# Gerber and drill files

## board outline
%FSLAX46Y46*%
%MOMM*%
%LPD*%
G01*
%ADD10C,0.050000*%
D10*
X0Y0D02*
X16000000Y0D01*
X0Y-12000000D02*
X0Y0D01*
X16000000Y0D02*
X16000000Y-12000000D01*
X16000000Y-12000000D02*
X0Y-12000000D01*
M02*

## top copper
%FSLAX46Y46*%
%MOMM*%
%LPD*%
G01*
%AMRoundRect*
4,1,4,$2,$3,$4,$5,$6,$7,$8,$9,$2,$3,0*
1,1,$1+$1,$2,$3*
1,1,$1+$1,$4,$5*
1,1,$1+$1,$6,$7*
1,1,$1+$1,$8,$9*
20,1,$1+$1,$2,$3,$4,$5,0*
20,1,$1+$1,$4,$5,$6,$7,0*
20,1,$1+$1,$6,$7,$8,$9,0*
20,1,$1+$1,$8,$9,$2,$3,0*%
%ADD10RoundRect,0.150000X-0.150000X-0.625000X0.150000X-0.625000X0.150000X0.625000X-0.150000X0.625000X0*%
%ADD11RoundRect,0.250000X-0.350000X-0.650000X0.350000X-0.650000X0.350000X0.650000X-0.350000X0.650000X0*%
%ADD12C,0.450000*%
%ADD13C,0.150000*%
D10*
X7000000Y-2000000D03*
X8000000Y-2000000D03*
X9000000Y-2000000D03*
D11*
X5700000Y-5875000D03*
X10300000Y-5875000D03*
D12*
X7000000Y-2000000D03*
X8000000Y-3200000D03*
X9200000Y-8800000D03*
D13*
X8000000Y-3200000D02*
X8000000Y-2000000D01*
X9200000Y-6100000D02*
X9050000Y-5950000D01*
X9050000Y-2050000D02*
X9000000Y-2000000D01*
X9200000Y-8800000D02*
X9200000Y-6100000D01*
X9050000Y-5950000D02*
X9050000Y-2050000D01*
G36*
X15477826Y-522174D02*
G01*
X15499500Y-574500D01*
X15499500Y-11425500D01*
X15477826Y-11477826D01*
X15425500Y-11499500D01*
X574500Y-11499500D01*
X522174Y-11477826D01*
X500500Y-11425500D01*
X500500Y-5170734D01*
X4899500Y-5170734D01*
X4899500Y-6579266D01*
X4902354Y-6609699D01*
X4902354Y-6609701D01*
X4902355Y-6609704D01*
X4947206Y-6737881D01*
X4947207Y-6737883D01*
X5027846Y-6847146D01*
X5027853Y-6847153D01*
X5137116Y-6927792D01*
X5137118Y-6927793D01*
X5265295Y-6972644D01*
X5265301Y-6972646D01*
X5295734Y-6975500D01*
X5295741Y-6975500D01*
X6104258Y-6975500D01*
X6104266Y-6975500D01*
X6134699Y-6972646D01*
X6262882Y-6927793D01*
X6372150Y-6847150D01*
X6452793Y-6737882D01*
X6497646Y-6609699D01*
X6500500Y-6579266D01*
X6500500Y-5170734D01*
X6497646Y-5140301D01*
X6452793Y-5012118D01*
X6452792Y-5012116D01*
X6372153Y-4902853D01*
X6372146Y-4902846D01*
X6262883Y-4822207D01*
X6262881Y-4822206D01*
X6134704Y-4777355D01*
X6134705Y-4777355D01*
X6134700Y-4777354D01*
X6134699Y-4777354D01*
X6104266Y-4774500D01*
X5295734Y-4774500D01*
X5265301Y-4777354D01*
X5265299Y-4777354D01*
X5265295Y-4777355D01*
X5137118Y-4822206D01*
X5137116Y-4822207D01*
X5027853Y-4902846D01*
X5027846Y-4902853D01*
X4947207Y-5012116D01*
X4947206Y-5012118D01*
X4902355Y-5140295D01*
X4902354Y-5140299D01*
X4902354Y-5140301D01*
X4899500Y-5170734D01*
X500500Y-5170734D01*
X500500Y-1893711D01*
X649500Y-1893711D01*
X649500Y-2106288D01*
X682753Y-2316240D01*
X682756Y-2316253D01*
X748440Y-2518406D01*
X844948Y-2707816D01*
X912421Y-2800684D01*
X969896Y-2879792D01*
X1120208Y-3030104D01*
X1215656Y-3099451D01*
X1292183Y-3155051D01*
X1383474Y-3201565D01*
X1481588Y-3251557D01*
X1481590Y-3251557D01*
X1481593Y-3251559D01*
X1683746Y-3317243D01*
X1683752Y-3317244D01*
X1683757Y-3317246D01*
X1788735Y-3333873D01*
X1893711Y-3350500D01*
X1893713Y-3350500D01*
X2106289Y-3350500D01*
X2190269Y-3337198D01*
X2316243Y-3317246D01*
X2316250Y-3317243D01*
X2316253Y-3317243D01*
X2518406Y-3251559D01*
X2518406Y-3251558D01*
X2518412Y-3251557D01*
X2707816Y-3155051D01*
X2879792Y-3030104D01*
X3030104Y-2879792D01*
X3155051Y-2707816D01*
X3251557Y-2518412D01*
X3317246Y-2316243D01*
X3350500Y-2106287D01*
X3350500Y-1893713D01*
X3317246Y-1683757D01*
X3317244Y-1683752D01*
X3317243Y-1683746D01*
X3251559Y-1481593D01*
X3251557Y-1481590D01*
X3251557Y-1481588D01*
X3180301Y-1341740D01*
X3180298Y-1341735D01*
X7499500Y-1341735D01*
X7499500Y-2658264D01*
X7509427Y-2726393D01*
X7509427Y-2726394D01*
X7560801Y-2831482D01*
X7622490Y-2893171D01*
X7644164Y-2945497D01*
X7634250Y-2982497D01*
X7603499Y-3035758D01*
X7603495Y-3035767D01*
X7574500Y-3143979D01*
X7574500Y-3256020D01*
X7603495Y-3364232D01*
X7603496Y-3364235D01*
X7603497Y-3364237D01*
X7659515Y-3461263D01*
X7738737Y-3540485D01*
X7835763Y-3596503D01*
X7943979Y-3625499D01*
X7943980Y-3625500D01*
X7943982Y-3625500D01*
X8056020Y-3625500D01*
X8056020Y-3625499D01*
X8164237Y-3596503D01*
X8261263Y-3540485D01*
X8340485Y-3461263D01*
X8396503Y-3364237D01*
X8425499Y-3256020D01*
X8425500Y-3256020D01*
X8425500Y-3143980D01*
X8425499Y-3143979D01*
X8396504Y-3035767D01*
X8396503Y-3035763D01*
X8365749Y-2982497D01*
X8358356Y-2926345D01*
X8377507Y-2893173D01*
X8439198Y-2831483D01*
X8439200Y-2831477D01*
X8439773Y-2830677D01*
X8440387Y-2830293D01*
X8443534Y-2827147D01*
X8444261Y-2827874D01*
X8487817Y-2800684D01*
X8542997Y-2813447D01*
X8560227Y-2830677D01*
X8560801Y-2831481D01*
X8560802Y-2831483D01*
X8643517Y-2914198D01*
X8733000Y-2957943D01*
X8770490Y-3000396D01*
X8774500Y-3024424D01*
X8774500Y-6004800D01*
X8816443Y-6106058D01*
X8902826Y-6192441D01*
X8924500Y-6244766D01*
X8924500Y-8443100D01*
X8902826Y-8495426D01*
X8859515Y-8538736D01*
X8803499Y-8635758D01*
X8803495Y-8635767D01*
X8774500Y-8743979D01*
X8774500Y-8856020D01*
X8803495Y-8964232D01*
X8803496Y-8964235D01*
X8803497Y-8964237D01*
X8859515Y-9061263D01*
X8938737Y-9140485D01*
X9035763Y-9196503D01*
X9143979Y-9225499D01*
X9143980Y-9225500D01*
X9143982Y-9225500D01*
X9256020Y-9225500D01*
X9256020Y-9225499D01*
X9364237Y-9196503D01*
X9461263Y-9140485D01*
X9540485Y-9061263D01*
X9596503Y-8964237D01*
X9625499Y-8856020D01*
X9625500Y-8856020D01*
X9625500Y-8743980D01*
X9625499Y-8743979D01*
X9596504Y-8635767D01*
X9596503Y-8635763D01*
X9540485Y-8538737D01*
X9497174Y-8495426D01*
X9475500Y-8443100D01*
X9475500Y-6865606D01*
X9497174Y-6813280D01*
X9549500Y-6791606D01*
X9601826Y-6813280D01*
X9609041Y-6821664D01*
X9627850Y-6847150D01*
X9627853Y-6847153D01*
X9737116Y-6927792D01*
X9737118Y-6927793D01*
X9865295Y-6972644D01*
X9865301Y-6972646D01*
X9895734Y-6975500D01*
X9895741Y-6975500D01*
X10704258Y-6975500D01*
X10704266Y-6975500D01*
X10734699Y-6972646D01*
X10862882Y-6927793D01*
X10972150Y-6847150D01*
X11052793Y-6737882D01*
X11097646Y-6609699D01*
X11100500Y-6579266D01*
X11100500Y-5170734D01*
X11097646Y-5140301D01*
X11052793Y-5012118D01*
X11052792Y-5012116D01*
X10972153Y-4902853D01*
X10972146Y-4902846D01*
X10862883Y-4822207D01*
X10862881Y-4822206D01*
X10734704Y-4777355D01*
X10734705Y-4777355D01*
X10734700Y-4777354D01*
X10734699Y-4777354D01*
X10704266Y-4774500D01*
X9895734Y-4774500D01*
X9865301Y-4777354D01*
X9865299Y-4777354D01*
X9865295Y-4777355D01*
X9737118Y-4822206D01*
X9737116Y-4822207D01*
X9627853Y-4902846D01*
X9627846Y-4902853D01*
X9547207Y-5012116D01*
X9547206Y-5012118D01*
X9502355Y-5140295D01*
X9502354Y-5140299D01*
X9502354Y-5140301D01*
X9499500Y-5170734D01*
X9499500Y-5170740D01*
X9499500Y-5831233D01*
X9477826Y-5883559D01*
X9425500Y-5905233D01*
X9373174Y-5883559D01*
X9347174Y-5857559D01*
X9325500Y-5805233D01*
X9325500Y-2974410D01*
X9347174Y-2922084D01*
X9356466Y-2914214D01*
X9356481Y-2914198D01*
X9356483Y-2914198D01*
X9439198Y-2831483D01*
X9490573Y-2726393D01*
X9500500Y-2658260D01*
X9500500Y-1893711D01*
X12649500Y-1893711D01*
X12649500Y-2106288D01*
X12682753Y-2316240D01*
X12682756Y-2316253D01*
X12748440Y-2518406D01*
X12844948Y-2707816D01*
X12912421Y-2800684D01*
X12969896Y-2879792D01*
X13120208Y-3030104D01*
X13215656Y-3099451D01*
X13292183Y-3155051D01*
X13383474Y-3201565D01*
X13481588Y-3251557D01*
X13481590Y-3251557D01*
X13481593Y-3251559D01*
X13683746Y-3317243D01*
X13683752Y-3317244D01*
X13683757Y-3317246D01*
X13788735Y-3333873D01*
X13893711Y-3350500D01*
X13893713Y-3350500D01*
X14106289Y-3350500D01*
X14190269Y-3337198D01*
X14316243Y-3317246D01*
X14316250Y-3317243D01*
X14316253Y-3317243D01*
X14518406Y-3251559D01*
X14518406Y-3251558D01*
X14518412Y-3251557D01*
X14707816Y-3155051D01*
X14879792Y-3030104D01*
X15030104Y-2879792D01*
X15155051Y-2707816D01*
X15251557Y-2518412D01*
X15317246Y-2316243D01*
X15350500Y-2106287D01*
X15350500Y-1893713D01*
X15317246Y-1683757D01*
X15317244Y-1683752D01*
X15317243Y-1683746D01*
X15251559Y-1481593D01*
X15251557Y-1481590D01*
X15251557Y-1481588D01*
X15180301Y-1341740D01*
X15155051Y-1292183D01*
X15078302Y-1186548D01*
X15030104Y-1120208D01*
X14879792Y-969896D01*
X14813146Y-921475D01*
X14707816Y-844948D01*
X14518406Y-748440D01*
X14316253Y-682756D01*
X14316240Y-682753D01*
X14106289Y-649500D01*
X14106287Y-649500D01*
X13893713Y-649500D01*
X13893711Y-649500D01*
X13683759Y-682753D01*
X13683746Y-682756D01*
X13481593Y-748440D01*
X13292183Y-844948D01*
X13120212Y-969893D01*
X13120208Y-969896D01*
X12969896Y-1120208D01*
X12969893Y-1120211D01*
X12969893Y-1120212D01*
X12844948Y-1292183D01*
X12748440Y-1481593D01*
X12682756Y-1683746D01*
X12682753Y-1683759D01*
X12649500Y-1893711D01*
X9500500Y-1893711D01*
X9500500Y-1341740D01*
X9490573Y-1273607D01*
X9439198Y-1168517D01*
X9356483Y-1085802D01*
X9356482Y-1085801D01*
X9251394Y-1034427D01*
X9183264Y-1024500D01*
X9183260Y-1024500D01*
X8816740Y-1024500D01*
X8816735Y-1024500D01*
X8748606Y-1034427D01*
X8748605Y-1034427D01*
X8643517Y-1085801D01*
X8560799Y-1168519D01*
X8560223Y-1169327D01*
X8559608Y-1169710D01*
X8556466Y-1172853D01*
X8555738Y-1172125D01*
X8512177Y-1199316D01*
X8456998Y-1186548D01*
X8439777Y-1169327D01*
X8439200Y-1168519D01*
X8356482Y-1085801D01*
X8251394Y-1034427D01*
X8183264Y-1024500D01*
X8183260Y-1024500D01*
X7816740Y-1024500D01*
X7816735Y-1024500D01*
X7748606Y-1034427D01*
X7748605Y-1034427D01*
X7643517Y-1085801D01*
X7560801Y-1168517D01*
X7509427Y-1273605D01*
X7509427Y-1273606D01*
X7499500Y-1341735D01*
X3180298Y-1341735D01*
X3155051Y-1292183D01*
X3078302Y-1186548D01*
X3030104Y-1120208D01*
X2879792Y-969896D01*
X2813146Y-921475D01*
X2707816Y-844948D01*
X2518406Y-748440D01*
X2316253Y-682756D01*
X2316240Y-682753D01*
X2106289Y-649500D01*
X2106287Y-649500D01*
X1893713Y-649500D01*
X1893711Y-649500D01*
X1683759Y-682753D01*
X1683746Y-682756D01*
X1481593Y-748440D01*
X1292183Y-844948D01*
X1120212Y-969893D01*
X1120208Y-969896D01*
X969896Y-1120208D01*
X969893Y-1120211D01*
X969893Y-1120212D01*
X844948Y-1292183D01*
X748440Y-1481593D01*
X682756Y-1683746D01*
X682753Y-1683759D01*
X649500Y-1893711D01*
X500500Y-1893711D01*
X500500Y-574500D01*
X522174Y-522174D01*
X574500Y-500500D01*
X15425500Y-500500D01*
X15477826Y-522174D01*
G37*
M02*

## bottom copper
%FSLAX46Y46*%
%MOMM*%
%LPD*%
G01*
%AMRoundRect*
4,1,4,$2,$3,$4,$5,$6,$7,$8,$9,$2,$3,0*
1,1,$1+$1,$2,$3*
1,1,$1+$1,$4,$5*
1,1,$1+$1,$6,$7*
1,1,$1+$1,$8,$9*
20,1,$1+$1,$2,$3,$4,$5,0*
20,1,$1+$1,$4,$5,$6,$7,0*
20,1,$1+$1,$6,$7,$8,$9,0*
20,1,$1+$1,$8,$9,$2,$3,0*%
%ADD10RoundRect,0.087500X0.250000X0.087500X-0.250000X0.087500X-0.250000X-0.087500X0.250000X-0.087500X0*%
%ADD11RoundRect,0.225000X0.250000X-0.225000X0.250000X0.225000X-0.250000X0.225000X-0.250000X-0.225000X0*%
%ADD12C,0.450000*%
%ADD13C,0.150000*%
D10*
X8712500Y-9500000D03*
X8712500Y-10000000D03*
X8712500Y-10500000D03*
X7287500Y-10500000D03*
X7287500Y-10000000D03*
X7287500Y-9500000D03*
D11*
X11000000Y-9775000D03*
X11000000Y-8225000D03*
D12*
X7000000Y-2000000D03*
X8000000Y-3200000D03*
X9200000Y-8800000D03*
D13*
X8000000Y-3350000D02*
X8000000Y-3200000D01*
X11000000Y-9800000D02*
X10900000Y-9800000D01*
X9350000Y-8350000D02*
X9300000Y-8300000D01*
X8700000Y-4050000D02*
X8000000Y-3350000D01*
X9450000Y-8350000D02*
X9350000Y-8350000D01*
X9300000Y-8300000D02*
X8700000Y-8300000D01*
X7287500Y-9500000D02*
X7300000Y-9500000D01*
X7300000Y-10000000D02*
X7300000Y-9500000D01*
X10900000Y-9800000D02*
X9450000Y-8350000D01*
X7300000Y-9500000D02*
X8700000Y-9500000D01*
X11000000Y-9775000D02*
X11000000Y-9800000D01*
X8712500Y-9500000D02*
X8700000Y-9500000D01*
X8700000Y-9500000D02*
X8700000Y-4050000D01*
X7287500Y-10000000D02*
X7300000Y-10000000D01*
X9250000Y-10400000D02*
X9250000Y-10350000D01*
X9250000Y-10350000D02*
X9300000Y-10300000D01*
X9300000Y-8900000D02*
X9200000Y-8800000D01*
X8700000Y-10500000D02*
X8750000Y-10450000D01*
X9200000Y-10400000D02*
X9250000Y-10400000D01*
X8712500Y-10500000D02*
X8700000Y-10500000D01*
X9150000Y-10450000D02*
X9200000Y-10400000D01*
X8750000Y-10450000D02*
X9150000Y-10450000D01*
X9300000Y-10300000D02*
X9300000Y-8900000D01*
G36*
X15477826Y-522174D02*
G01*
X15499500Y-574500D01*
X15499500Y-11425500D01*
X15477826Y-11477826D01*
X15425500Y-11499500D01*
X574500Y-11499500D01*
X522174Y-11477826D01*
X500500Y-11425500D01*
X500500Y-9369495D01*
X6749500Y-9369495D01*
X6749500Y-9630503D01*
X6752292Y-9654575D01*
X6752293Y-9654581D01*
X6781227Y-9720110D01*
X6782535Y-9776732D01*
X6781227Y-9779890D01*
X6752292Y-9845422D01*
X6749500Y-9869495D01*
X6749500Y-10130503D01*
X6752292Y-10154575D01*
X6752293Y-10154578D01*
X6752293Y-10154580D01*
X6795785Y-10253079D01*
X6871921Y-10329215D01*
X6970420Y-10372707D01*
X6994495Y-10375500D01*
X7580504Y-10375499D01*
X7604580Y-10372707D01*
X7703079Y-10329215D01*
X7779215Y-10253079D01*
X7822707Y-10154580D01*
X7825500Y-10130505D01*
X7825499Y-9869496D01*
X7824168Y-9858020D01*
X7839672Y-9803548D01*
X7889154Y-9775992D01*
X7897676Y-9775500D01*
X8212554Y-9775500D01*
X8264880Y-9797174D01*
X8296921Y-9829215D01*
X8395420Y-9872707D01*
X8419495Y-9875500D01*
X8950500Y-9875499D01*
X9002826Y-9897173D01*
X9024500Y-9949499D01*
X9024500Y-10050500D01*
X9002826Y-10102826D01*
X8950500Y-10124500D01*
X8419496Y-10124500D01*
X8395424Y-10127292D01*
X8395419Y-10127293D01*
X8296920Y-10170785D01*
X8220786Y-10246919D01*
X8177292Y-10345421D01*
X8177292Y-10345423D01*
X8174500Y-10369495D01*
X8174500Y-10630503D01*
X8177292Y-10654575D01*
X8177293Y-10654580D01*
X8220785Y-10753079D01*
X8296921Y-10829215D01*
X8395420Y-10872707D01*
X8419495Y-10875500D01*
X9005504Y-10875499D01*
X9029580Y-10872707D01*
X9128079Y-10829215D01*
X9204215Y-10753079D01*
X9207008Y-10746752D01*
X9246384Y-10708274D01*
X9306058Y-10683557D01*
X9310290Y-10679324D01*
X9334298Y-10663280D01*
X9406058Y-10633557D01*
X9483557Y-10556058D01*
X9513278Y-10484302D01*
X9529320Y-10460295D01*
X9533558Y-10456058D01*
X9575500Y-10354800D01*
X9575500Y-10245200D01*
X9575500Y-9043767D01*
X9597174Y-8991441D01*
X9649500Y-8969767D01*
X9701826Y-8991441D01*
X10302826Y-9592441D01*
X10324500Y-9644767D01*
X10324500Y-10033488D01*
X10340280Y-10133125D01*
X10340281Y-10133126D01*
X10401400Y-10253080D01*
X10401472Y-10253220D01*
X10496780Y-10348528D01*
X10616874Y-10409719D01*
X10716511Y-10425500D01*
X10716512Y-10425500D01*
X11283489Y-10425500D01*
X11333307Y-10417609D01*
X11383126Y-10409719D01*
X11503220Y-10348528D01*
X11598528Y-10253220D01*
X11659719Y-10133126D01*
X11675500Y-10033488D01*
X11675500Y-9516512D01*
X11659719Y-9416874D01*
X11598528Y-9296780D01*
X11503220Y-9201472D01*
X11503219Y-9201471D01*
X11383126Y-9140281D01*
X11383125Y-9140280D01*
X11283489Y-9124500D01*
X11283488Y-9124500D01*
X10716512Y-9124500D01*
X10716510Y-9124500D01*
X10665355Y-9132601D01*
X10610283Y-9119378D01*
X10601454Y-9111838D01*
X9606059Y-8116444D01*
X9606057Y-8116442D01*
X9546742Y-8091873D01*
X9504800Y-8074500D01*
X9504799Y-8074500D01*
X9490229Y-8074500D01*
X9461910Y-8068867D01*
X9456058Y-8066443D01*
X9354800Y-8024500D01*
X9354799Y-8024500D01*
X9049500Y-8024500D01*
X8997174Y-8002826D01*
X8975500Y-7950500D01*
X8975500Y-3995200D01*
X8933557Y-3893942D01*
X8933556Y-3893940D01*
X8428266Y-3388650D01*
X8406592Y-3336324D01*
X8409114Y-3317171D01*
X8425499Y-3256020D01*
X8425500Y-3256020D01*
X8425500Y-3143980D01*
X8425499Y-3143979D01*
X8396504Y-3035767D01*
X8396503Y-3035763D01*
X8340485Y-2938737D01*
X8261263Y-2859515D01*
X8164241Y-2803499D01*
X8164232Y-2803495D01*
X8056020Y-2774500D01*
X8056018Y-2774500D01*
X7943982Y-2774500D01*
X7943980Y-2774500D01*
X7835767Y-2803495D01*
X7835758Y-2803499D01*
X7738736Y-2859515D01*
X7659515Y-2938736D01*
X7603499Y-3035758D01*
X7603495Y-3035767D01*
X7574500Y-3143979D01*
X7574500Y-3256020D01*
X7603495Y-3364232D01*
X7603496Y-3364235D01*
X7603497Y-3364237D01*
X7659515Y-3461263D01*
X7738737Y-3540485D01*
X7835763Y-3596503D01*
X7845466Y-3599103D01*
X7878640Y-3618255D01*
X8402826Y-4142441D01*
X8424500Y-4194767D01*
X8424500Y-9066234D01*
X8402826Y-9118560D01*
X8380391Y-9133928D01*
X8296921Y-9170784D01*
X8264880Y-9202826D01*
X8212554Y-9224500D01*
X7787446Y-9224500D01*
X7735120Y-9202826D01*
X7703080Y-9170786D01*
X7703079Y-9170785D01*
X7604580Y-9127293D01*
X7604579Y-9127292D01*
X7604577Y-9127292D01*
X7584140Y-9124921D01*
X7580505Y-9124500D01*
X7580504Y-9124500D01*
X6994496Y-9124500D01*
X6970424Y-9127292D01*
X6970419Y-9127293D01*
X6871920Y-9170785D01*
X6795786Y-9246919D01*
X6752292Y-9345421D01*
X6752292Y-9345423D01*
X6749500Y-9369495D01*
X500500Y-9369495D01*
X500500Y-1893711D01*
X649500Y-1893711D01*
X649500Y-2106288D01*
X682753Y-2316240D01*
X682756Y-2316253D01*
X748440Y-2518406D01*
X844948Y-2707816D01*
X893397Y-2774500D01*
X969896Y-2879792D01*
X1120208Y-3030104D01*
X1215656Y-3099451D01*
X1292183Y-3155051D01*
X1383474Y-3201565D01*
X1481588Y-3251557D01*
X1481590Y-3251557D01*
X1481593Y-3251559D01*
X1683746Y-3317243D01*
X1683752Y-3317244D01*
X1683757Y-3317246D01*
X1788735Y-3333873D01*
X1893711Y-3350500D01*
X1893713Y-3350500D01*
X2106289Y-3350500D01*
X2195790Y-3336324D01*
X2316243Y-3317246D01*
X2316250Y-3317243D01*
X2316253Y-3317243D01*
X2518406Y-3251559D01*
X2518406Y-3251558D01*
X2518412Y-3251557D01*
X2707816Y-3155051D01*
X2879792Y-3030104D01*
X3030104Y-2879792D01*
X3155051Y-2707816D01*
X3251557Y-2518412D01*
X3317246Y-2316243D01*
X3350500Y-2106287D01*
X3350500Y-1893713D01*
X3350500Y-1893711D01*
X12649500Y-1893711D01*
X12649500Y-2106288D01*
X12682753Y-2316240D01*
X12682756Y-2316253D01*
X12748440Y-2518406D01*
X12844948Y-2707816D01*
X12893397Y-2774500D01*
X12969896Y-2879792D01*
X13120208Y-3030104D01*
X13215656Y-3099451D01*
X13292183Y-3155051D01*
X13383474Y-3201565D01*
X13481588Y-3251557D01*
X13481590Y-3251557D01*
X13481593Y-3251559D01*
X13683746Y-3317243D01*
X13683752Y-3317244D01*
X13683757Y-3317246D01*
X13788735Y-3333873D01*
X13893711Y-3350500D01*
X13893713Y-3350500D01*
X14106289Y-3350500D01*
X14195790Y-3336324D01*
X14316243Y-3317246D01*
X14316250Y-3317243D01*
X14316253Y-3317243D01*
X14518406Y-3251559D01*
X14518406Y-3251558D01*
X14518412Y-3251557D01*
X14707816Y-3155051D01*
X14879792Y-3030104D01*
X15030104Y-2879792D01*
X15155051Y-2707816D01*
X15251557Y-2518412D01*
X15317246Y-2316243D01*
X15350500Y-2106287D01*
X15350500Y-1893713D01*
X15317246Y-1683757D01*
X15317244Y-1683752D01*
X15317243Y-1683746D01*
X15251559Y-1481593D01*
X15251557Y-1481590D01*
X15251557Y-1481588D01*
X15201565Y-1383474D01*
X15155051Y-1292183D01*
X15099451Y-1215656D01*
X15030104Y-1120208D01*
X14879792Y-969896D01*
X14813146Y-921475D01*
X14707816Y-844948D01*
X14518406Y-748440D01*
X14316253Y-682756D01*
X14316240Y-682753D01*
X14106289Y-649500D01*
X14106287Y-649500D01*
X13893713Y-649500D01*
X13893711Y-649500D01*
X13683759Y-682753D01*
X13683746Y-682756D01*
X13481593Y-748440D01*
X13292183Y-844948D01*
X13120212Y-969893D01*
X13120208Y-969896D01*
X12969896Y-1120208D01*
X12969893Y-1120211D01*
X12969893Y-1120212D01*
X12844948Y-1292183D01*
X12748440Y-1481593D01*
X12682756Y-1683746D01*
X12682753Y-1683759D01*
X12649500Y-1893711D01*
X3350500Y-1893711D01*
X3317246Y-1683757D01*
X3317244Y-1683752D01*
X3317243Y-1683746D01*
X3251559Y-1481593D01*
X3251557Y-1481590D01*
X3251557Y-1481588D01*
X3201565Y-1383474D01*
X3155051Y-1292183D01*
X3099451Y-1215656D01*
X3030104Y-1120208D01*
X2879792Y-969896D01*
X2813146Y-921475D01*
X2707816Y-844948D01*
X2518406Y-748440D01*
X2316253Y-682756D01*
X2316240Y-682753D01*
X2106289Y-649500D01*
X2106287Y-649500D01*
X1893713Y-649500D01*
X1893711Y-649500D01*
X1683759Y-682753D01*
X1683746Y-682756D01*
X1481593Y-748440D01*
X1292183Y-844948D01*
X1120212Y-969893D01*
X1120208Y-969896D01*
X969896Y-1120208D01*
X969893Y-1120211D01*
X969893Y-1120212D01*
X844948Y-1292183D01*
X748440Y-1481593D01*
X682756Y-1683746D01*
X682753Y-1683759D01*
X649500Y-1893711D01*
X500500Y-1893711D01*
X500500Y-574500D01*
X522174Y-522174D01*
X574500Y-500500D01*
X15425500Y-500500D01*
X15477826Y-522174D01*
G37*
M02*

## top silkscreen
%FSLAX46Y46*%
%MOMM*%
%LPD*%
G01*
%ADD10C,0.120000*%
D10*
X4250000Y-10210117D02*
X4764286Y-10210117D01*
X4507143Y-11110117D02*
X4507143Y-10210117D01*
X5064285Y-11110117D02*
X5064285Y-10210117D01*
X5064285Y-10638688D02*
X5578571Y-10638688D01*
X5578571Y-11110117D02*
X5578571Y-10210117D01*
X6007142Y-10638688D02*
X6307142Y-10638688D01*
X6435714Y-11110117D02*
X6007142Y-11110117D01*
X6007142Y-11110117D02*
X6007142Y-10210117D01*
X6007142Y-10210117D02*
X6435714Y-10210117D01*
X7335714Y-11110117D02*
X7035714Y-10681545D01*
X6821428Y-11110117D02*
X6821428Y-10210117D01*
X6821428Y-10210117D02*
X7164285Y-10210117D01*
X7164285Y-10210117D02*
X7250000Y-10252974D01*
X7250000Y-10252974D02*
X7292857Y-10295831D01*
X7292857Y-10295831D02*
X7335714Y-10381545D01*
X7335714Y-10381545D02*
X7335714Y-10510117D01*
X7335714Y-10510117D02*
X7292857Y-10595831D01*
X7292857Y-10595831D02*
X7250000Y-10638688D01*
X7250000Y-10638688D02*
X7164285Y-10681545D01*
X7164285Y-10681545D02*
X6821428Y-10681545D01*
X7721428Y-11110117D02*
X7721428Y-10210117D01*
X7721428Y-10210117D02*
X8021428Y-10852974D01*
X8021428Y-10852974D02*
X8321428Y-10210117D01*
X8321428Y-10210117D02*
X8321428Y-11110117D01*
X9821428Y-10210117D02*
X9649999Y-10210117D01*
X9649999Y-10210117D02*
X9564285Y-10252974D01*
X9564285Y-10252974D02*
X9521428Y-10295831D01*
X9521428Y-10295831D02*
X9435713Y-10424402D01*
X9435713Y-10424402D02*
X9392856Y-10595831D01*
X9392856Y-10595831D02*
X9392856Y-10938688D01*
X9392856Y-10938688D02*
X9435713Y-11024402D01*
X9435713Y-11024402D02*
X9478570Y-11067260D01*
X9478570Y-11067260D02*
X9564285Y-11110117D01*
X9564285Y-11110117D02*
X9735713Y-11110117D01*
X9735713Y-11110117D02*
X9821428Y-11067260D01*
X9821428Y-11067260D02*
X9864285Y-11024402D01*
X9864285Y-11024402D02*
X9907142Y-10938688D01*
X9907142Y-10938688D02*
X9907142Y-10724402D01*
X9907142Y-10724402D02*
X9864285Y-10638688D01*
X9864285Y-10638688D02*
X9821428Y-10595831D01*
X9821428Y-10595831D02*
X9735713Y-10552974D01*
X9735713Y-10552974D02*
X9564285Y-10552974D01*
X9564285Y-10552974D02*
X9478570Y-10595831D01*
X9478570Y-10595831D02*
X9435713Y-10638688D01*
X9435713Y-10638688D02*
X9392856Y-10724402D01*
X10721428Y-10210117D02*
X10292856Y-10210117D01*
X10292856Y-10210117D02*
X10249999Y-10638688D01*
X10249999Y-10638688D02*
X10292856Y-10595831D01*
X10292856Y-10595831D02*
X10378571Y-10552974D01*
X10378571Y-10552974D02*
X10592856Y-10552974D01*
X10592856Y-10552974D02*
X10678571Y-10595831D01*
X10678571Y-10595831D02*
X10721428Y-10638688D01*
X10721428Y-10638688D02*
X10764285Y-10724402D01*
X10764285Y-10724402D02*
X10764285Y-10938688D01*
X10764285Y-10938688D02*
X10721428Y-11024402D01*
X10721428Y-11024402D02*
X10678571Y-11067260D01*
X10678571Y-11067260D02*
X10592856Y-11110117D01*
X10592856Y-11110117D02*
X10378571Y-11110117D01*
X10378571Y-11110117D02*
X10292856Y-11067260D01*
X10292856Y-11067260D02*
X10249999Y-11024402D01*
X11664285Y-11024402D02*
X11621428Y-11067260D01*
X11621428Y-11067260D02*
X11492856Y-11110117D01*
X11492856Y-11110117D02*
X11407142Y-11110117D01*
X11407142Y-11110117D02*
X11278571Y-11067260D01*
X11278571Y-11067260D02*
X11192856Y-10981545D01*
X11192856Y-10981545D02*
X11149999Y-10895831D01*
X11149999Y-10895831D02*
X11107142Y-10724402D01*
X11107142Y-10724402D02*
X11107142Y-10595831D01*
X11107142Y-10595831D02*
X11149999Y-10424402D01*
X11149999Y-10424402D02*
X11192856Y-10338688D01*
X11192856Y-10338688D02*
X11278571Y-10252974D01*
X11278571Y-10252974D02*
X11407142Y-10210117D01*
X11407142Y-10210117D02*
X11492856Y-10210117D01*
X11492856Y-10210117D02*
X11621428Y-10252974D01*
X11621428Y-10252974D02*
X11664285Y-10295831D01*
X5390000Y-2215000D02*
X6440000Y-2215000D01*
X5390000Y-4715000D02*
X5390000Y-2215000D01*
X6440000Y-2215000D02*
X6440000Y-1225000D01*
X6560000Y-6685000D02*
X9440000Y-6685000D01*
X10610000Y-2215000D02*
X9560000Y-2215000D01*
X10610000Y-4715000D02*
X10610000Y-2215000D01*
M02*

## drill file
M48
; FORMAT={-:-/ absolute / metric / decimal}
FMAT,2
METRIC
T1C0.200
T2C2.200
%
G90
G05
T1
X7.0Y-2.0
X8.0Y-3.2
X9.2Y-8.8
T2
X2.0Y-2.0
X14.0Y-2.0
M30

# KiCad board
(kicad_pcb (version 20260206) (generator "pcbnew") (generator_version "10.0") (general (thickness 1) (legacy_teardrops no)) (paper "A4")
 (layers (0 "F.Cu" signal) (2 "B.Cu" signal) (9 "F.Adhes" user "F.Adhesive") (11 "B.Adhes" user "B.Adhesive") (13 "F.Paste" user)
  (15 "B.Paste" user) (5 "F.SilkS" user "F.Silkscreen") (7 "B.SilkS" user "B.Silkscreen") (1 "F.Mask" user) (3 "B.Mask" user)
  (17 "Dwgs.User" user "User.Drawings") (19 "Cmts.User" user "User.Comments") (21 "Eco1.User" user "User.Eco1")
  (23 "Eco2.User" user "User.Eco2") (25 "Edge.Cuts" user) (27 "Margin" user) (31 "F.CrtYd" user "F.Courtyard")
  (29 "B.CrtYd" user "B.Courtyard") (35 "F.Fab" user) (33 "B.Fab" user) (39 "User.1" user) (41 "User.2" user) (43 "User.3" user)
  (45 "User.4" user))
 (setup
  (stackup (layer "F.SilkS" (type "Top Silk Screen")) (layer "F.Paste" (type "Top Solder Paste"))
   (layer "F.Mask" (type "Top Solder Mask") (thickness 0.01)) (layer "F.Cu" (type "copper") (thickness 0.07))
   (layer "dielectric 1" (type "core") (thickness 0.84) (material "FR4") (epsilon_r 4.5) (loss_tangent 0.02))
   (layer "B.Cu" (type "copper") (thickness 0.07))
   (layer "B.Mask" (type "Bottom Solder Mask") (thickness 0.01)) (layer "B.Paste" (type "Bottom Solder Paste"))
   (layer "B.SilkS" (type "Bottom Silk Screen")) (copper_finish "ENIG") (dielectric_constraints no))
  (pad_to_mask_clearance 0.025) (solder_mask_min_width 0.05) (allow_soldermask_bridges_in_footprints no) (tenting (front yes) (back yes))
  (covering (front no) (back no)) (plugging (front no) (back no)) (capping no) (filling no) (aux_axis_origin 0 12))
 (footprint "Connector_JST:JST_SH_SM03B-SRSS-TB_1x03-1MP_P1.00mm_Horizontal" (layer "F.Cu") (at 8 4)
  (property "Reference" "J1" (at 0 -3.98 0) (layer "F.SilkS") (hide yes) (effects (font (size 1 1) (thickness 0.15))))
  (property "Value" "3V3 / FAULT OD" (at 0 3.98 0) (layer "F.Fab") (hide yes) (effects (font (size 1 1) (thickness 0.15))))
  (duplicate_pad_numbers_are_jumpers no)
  (fp_line (start -2.61 -1.785) (end -1.56 -1.785) (stroke (width 0.12) (type solid)) (layer "F.SilkS"))
  (fp_line (start -2.61 0.715) (end -2.61 -1.785) (stroke (width 0.12) (type solid)) (layer "F.SilkS"))
  (fp_line (start -1.56 -1.785) (end -1.56 -2.775) (stroke (width 0.12) (type solid)) (layer "F.SilkS"))
  (fp_line (start -1.44 2.685) (end 1.44 2.685) (stroke (width 0.12) (type solid)) (layer "F.SilkS"))
  (fp_line (start 2.61 -1.785) (end 1.56 -1.785) (stroke (width 0.12) (type solid)) (layer "F.SilkS"))
  (fp_line (start 2.61 0.715) (end 2.61 -1.785) (stroke (width 0.12) (type solid)) (layer "F.SilkS"))
  (pad "1" smd roundrect (at -1 -2) (size 0.6 1.55) (layers "F.Cu" "F.Mask" "F.Paste") (roundrect_rratio 0.25) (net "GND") (zone_connect 2))
  (pad "2" smd roundrect (at 0 -2) (size 0.6 1.55) (layers "F.Cu" "F.Mask" "F.Paste") (roundrect_rratio 0.25) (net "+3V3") (zone_connect 2))
  (pad "3" smd roundrect (at 1 -2) (size 0.6 1.55) (layers "F.Cu" "F.Mask" "F.Paste") (roundrect_rratio 0.25) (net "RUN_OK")
   (zone_connect 2))
  (pad "MP" smd roundrect (at -2.3 1.875) (size 1.2 1.8) (layers "F.Cu" "F.Mask" "F.Paste") (roundrect_rratio 0.208333) (zone_connect 2))
  (pad "MP" smd roundrect (at 2.3 1.875) (size 1.2 1.8) (layers "F.Cu" "F.Mask" "F.Paste") (roundrect_rratio 0.208333) (zone_connect 2)))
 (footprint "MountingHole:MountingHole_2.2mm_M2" (layer "F.Cu") (at 14 2)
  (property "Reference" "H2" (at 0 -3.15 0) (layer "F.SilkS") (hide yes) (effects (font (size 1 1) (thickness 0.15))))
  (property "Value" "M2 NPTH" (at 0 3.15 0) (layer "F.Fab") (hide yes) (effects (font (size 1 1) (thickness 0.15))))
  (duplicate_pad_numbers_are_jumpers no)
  (pad "" np_thru_hole circle (at 0 0) (size 2.2 2.2) (drill 2.2) (layers "*.Cu" "*.Mask") (zone_connect 2)))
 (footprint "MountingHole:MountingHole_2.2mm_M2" (layer "F.Cu") (at 2 2)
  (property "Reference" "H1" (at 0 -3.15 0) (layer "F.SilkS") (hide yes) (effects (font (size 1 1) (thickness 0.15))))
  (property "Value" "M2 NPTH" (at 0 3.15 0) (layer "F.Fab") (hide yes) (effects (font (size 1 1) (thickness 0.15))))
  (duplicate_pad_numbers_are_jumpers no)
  (pad "" np_thru_hole circle (at 0 0) (size 2.2 2.2) (drill 2.2) (layers "*.Cu" "*.Mask") (zone_connect 2)))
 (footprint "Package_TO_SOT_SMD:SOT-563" (layer "B.Cu") (at 8 10 180)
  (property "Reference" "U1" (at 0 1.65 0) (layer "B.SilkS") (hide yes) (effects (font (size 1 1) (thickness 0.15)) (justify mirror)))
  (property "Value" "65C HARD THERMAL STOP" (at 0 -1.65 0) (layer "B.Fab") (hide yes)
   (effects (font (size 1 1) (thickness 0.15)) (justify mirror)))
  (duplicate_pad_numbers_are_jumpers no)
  (pad "1" smd roundrect (at -0.7125 0.5 180) (size 0.675 0.35) (layers "B.Cu" "B.Mask" "B.Paste") (roundrect_rratio 0.25) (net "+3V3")
   (zone_connect 2))
  (pad "2" smd roundrect (at -0.7125 0 180) (size 0.675 0.35) (layers "B.Cu" "B.Mask" "B.Paste") (roundrect_rratio 0.25) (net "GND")
   (zone_connect 2))
  (pad "3" smd roundrect (at -0.7125 -0.5 180) (size 0.675 0.35) (layers "B.Cu" "B.Mask" "B.Paste") (roundrect_rratio 0.25) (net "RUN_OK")
   (zone_connect 2))
  (pad "4" smd roundrect (at 0.7125 -0.5 180) (size 0.675 0.35) (layers "B.Cu" "B.Mask" "B.Paste") (roundrect_rratio 0.25) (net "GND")
   (zone_connect 2))
  (pad "5" smd roundrect (at 0.7125 0 180) (size 0.675 0.35) (layers "B.Cu" "B.Mask" "B.Paste") (roundrect_rratio 0.25) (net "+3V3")
   (zone_connect 2))
  (pad "6" smd roundrect (at 0.7125 0.5 180) (size 0.675 0.35) (layers "B.Cu" "B.Mask" "B.Paste") (roundrect_rratio 0.25) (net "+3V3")
   (zone_connect 2)))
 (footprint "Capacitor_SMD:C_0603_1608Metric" (layer "B.Cu") (at 11 9 90)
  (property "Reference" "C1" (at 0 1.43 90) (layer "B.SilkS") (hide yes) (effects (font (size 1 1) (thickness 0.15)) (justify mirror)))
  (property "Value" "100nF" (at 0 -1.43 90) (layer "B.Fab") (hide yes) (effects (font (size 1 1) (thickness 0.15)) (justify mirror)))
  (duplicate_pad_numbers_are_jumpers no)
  (pad "1" smd roundrect (at -0.775 0 90) (size 0.9 0.95) (layers "B.Cu" "B.Mask" "B.Paste") (roundrect_rratio 0.25) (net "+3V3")
   (zone_connect 2))
  (pad "2" smd roundrect (at 0.775 0 90) (size 0.9 0.95) (layers "B.Cu" "B.Mask" "B.Paste") (roundrect_rratio 0.25) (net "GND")
   (zone_connect 2)))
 (gr_line (start 0 0) (end 16 0) (stroke (width 0.05) (type default)) (layer "Edge.Cuts"))
 (gr_line (start 0 12) (end 0 0) (stroke (width 0.05) (type default)) (layer "Edge.Cuts"))
 (gr_line (start 16 0) (end 16 12) (stroke (width 0.05) (type default)) (layer "Edge.Cuts"))
 (gr_line (start 16 12) (end 0 12) (stroke (width 0.05) (type default)) (layer "Edge.Cuts"))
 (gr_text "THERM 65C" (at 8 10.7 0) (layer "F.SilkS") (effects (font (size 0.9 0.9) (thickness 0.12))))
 (via (at 7 2) (size 0.45) (drill 0.2) (layers "F.Cu" "B.Cu") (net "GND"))
 (segment (start 8 3.2) (end 8 2) (width 0.15) (layer "F.Cu") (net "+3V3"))
 (via (at 8 3.2) (size 0.45) (drill 0.2) (layers "F.Cu" "B.Cu") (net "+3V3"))
 (segment (start 8 3.35) (end 8 3.2) (width 0.15) (layer "B.Cu") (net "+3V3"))
 (segment (start 11 9.8) (end 10.9 9.8) (width 0.15) (layer "B.Cu") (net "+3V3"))
 (segment (start 9.35 8.35) (end 9.3 8.3) (width 0.15) (layer "B.Cu") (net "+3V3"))
 (segment (start 8.7 4.05) (end 8 3.35) (width 0.15) (layer "B.Cu") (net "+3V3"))
 (segment (start 9.45 8.35) (end 9.35 8.35) (width 0.15) (layer "B.Cu") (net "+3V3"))
 (segment (start 9.3 8.3) (end 8.7 8.3) (width 0.15) (layer "B.Cu") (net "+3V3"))
 (segment (start 7.2875 9.5) (end 7.3 9.5) (width 0.15) (layer "B.Cu") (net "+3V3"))
 (segment (start 7.3 10) (end 7.3 9.5) (width 0.15) (layer "B.Cu") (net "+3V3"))
 (segment (start 10.9 9.8) (end 9.45 8.35) (width 0.15) (layer "B.Cu") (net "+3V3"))
 (segment (start 7.3 9.5) (end 8.7 9.5) (width 0.15) (layer "B.Cu") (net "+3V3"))
 (segment (start 11 9.775) (end 11 9.8) (width 0.15) (layer "B.Cu") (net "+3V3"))
 (segment (start 8.7125 9.5) (end 8.7 9.5) (width 0.15) (layer "B.Cu") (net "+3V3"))
 (segment (start 8.7 9.5) (end 8.7 4.05) (width 0.15) (layer "B.Cu") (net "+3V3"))
 (segment (start 7.2875 10) (end 7.3 10) (width 0.15) (layer "B.Cu") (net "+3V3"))
 (segment (start 9.2 6.1) (end 9.05 5.95) (width 0.15) (layer "F.Cu") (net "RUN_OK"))
 (segment (start 9.05 2.05) (end 9 2) (width 0.15) (layer "F.Cu") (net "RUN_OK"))
 (segment (start 9.2 8.8) (end 9.2 6.1) (width 0.15) (layer "F.Cu") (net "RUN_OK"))
 (segment (start 9.05 5.95) (end 9.05 2.05) (width 0.15) (layer "F.Cu") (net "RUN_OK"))
 (via (at 9.2 8.8) (size 0.45) (drill 0.2) (layers "F.Cu" "B.Cu") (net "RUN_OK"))
 (segment (start 9.25 10.4) (end 9.25 10.35) (width 0.15) (layer "B.Cu") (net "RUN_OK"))
 (segment (start 9.25 10.35) (end 9.3 10.3) (width 0.15) (layer "B.Cu") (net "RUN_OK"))
 (segment (start 9.3 8.9) (end 9.2 8.8) (width 0.15) (layer "B.Cu") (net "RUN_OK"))
 (segment (start 8.7 10.5) (end 8.75 10.45) (width 0.15) (layer "B.Cu") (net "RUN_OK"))
 (segment (start 9.2 10.4) (end 9.25 10.4) (width 0.15) (layer "B.Cu") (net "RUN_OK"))
 (segment (start 8.7125 10.5) (end 8.7 10.5) (width 0.15) (layer "B.Cu") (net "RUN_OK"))
 (segment (start 9.15 10.45) (end 9.2 10.4) (width 0.15) (layer "B.Cu") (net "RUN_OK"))
 (segment (start 8.75 10.45) (end 9.15 10.45) (width 0.15) (layer "B.Cu") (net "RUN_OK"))
 (segment (start 9.3 10.3) (end 9.3 8.9) (width 0.15) (layer "B.Cu") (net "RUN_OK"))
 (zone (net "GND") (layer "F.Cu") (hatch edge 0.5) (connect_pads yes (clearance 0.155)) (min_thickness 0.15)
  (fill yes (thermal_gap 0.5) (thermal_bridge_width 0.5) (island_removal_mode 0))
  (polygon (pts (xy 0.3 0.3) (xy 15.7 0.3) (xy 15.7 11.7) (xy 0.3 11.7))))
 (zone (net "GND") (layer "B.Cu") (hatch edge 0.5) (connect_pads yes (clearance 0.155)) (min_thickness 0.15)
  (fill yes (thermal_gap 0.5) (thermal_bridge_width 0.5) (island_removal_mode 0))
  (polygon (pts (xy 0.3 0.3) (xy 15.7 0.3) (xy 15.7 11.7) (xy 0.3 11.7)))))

